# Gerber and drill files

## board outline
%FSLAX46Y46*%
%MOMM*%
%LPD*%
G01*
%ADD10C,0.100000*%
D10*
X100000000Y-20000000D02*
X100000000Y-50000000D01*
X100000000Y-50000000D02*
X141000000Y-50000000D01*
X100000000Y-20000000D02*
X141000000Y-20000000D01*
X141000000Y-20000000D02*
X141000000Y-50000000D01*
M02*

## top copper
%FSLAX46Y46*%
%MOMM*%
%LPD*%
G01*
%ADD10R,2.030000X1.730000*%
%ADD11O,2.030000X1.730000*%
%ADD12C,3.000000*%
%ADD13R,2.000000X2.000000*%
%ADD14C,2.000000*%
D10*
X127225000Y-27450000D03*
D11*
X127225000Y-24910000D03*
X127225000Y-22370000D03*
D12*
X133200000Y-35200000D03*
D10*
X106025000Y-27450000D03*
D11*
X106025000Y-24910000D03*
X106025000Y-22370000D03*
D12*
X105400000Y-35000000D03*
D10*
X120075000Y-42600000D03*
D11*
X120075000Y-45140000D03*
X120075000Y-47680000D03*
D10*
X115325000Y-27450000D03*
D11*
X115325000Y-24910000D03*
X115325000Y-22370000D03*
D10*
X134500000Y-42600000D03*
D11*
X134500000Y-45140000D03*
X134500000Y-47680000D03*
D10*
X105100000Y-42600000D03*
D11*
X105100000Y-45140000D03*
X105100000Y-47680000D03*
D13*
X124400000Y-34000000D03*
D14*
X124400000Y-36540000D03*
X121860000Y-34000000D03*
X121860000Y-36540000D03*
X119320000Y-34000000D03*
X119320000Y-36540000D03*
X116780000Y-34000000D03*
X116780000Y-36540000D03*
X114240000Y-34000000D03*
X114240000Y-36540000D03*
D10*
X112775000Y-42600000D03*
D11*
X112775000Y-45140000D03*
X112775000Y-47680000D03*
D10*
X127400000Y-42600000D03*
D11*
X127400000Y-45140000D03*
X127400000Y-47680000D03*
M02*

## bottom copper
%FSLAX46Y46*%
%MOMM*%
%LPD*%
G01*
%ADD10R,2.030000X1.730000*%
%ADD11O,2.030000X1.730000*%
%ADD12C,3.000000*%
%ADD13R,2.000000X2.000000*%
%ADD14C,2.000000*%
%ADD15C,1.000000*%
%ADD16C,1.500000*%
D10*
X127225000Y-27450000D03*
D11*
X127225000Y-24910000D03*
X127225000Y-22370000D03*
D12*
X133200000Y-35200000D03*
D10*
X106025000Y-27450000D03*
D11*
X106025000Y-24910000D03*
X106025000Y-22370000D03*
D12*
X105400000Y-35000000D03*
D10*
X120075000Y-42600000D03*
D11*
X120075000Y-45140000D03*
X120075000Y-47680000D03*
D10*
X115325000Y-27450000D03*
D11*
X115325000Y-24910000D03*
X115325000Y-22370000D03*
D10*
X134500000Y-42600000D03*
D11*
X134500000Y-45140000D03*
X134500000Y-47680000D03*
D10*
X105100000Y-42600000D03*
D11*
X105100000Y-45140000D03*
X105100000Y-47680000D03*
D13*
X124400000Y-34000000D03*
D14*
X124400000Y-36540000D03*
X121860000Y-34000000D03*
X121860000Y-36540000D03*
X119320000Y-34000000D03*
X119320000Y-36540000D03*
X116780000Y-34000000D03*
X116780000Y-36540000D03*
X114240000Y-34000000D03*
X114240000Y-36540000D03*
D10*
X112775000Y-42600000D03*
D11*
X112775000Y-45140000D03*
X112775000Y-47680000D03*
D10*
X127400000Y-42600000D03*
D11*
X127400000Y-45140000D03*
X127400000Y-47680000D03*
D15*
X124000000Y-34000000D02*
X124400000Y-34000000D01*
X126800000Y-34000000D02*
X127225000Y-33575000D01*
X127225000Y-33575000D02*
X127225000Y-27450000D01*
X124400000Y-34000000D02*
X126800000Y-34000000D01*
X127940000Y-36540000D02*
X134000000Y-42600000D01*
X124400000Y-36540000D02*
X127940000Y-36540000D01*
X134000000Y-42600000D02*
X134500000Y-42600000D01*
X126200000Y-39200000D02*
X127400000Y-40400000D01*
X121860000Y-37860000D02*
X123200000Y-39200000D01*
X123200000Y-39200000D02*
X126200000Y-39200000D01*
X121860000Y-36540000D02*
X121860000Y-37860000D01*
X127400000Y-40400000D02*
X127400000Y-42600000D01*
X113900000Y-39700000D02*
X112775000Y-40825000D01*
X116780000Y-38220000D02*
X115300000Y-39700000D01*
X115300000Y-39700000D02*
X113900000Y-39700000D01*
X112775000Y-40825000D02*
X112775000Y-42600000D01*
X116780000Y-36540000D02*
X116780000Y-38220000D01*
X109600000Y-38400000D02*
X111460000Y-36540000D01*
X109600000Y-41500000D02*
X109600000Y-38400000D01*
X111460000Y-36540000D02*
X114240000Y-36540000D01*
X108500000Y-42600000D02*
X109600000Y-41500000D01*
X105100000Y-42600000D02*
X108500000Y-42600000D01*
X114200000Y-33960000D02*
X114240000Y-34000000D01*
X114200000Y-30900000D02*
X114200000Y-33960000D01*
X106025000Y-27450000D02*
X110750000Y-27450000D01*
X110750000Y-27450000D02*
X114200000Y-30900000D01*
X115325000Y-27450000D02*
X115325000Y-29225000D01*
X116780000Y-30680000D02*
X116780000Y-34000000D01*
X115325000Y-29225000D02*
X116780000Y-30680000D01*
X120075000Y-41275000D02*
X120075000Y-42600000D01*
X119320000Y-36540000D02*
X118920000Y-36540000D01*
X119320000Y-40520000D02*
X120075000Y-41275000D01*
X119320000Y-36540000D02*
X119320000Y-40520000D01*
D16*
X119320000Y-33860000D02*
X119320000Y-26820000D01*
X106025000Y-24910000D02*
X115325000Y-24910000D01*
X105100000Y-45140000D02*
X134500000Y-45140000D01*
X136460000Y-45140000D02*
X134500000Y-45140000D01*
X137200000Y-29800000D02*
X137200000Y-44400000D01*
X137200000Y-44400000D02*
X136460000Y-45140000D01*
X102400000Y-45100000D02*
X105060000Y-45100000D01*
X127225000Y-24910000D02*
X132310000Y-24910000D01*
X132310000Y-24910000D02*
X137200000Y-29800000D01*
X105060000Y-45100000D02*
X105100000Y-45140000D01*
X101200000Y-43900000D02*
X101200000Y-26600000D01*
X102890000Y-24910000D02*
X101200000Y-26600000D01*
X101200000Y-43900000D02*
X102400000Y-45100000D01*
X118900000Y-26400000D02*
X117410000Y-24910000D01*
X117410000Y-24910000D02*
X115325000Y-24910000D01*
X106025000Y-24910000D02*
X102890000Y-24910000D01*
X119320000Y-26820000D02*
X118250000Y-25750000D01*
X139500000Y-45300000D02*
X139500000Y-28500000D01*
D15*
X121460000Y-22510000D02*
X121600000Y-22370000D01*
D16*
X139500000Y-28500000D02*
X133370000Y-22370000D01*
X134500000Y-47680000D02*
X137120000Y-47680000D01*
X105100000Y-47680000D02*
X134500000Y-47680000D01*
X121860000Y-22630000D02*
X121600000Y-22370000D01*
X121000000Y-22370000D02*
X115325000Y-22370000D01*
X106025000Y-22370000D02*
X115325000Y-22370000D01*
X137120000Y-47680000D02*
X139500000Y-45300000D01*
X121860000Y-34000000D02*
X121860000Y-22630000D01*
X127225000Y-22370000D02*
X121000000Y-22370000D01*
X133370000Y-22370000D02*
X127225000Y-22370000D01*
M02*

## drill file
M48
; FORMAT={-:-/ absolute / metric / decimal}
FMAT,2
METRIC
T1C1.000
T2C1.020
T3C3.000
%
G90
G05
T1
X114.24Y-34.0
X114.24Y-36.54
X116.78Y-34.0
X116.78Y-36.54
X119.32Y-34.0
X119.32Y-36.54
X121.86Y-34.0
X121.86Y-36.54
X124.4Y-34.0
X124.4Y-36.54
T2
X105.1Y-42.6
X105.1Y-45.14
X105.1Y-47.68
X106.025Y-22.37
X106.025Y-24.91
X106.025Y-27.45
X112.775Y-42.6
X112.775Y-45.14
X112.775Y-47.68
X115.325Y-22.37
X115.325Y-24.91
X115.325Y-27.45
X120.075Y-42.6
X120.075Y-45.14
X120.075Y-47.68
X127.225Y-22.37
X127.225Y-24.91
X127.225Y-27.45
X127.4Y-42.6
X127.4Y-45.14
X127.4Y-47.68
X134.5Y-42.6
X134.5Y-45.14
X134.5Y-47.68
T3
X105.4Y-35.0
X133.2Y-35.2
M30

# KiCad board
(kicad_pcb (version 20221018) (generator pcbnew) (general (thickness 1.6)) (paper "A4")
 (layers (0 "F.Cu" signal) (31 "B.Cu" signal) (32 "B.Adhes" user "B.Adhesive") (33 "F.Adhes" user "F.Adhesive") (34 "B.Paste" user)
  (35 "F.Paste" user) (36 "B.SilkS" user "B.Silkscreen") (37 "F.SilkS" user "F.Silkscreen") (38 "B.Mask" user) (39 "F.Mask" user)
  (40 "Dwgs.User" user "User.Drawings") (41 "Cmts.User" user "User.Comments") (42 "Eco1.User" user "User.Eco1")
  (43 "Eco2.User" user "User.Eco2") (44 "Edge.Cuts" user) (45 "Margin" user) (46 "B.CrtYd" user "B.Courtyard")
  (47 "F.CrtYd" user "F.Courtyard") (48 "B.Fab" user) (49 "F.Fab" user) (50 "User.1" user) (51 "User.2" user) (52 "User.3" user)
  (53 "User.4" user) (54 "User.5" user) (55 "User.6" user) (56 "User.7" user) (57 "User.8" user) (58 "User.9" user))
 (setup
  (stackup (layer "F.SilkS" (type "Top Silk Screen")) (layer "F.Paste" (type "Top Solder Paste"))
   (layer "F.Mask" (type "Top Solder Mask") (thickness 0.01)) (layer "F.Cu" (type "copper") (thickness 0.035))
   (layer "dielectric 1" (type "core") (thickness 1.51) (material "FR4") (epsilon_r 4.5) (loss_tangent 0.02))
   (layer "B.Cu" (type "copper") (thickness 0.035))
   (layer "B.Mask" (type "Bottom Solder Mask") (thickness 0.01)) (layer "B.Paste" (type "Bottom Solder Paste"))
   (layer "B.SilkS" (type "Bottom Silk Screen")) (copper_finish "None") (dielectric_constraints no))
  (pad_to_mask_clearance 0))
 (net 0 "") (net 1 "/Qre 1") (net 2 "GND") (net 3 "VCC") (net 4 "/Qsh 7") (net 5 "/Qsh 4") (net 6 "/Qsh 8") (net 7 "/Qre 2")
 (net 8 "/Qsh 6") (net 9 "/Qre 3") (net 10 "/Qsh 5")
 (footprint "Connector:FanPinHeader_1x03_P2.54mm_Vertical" (layer "F.Cu") (at 127.225 27.45 90)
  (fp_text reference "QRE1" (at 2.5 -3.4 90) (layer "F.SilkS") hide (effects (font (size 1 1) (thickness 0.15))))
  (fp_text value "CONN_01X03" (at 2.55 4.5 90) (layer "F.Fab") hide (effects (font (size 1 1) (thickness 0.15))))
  (pad "1" thru_hole rect (at 0 0 180) (size 2.03 1.73) (drill 1.02) (layers "*.Cu" "*.Mask") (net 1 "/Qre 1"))
  (pad "2" thru_hole oval (at 2.54 0 180) (size 2.03 1.73) (drill 1.02) (layers "*.Cu" "*.Mask") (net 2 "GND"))
  (pad "3" thru_hole oval (at 5.08 0 180) (size 2.03 1.73) (drill 1.02) (layers "*.Cu" "*.Mask") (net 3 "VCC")))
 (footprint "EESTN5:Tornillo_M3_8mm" (layer "F.Cu") (at 133.2 35.2)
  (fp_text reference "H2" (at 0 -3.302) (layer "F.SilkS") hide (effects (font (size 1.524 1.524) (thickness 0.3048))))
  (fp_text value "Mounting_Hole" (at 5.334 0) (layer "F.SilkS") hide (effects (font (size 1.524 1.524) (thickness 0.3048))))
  (pad "1" thru_hole circle (at 0 0) (size 3 3) (drill 3) (layers "*.Cu" "F.SilkS")))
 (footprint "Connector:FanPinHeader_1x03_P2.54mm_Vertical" (layer "F.Cu") (at 106.025 27.45 90)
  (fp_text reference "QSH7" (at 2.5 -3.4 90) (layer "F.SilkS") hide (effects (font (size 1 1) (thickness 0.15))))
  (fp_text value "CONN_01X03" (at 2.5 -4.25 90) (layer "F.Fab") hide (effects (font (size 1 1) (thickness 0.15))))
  (pad "1" thru_hole rect (at 0 0 180) (size 2.03 1.73) (drill 1.02) (layers "*.Cu" "*.Mask") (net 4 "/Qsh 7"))
  (pad "2" thru_hole oval (at 2.54 0 180) (size 2.03 1.73) (drill 1.02) (layers "*.Cu" "*.Mask") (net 2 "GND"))
  (pad "3" thru_hole oval (at 5.08 0 180) (size 2.03 1.73) (drill 1.02) (layers "*.Cu" "*.Mask") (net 3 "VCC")))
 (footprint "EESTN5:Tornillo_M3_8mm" (layer "F.Cu") (at 105.4 35)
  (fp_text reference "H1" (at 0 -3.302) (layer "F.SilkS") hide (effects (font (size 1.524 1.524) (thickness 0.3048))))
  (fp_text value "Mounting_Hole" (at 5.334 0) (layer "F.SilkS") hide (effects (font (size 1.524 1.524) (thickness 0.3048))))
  (pad "1" thru_hole circle (at 0 0) (size 3 3) (drill 3) (layers "*.Cu" "F.SilkS")))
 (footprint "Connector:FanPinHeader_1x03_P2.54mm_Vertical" (layer "F.Cu") (at 120.075 42.6 -90)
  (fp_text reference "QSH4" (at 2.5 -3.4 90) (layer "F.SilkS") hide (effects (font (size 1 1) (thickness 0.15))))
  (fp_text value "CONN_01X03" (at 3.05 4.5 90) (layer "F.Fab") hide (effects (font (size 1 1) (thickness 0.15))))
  (pad "1" thru_hole rect (at 0 0) (size 2.03 1.73) (drill 1.02) (layers "*.Cu" "*.Mask") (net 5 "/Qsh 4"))
  (pad "2" thru_hole oval (at 2.54 0) (size 2.03 1.73) (drill 1.02) (layers "*.Cu" "*.Mask") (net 2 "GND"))
  (pad "3" thru_hole oval (at 5.08 0) (size 2.03 1.73) (drill 1.02) (layers "*.Cu" "*.Mask") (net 3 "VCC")))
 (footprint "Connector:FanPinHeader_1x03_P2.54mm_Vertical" (layer "F.Cu") (at 115.325 27.45 90)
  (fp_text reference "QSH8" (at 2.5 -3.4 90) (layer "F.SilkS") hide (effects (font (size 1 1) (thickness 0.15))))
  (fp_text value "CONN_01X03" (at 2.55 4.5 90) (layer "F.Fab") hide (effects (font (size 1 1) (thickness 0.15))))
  (pad "1" thru_hole rect (at 0 0 180) (size 2.03 1.73) (drill 1.02) (layers "*.Cu" "*.Mask") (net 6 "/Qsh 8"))
  (pad "2" thru_hole oval (at 2.54 0 180) (size 2.03 1.73) (drill 1.02) (layers "*.Cu" "*.Mask") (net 2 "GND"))
  (pad "3" thru_hole oval (at 5.08 0 180) (size 2.03 1.73) (drill 1.02) (layers "*.Cu" "*.Mask") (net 3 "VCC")))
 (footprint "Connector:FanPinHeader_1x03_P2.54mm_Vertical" (layer "F.Cu") (at 134.5 42.6 -90)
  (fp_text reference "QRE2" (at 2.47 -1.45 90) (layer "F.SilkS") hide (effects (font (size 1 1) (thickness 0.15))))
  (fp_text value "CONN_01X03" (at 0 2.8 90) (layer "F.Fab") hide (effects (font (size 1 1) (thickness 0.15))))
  (pad "1" thru_hole rect (at 0 0) (size 2.03 1.73) (drill 1.02) (layers "*.Cu" "*.Mask") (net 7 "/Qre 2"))
  (pad "2" thru_hole oval (at 2.54 0) (size 2.03 1.73) (drill 1.02) (layers "*.Cu" "*.Mask") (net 2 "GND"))
  (pad "3" thru_hole oval (at 5.08 0) (size 2.03 1.73) (drill 1.02) (layers "*.Cu" "*.Mask") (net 3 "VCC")))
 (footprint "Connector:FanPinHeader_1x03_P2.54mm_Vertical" (layer "F.Cu") (at 105.1 42.6 -90)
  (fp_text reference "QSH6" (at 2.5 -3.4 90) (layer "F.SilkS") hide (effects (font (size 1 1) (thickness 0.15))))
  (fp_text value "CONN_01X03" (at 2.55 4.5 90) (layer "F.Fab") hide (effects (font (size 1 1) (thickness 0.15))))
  (pad "1" thru_hole rect (at 0 0) (size 2.03 1.73) (drill 1.02) (layers "*.Cu" "*.Mask") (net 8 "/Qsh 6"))
  (pad "2" thru_hole oval (at 2.54 0) (size 2.03 1.73) (drill 1.02) (layers "*.Cu" "*.Mask") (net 2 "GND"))
  (pad "3" thru_hole oval (at 5.08 0) (size 2.03 1.73) (drill 1.02) (layers "*.Cu" "*.Mask") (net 3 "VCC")))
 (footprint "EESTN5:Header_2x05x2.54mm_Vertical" (layer "F.Cu") (at 119.32 35.27 180)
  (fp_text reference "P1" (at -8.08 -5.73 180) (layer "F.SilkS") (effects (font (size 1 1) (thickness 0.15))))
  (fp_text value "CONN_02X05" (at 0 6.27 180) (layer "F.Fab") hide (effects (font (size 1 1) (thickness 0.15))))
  (pad "1" thru_hole rect (at -5.08 1.27 180) (size 2 2) (drill 1) (layers "*.Cu" "*.Mask") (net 1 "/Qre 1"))
  (pad "2" thru_hole circle (at -5.08 -1.27 180) (size 2 2) (drill 1) (layers "*.Cu" "*.Mask") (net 7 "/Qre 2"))
  (pad "3" thru_hole circle (at -2.54 1.27 180) (size 2 2) (drill 1) (layers "*.Cu" "*.Mask") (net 3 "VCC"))
  (pad "4" thru_hole circle (at -2.54 -1.27 180) (size 2 2) (drill 1) (layers "*.Cu" "*.Mask") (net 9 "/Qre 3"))
  (pad "5" thru_hole circle (at 0 1.27 180) (size 2 2) (drill 1) (layers "*.Cu" "*.Mask") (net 2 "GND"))
  (pad "6" thru_hole circle (at 0 -1.27 180) (size 2 2) (drill 1) (layers "*.Cu" "*.Mask") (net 5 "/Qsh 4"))
  (pad "7" thru_hole circle (at 2.54 1.27 180) (size 2 2) (drill 1) (layers "*.Cu" "*.Mask") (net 6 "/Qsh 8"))
  (pad "8" thru_hole circle (at 2.54 -1.27 180) (size 2 2) (drill 1) (layers "*.Cu" "*.Mask") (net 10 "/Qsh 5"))
  (pad "9" thru_hole circle (at 5.08 1.27 180) (size 2 2) (drill 1) (layers "*.Cu" "*.Mask") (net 4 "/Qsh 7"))
  (pad "10" thru_hole circle (at 5.08 -1.27 180) (size 2 2) (drill 1) (layers "*.Cu" "*.Mask") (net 8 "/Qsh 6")))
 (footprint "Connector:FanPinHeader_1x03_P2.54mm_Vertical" (layer "F.Cu") (at 112.775 42.6 -90)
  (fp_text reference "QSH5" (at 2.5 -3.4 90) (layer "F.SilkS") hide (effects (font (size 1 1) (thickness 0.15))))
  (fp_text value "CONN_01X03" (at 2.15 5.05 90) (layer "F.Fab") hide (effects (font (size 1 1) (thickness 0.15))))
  (pad "1" thru_hole rect (at 0 0) (size 2.03 1.73) (drill 1.02) (layers "*.Cu" "*.Mask") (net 10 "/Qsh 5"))
  (pad "2" thru_hole oval (at 2.54 0) (size 2.03 1.73) (drill 1.02) (layers "*.Cu" "*.Mask") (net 2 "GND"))
  (pad "3" thru_hole oval (at 5.08 0) (size 2.03 1.73) (drill 1.02) (layers "*.Cu" "*.Mask") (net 3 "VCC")))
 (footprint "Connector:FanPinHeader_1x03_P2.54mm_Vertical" (layer "F.Cu") (at 127.4 42.6 -90)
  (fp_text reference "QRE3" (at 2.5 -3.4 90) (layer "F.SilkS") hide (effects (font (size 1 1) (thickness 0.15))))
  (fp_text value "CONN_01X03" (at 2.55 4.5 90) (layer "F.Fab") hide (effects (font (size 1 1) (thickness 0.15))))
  (pad "1" thru_hole rect (at 0 0) (size 2.03 1.73) (drill 1.02) (layers "*.Cu" "*.Mask") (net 9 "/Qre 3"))
  (pad "2" thru_hole oval (at 2.54 0) (size 2.03 1.73) (drill 1.02) (layers "*.Cu" "*.Mask") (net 2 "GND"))
  (pad "3" thru_hole oval (at 5.08 0) (size 2.03 1.73) (drill 1.02) (layers "*.Cu" "*.Mask") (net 3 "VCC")))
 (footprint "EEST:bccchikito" (layer "B.Cu") (at 138.6 22.6 180)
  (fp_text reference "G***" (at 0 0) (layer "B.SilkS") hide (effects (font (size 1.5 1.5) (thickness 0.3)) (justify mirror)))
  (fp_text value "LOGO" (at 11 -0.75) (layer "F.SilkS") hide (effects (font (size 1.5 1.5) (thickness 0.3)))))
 (gr_line (start 100 20) (end 100 50) (stroke (width 0.1) (type default)) (layer "Edge.Cuts"))
 (gr_line (start 100 50) (end 141 50) (stroke (width 0.1) (type default)) (layer "Edge.Cuts"))
 (gr_line (start 100 20) (end 141 20) (stroke (width 0.1) (type default)) (layer "Edge.Cuts"))
 (gr_line (start 141 20) (end 141 50) (stroke (width 0.1) (type default)) (layer "Edge.Cuts"))
 (segment (start 124 34) (end 124.4 34) (width 1) (layer "B.Cu") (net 1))
 (segment (start 126.8 34) (end 127.225 33.575) (width 1) (layer "B.Cu") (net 1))
 (segment (start 127.225 33.575) (end 127.225 27.45) (width 1) (layer "B.Cu") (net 1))
 (segment (start 124.4 34) (end 126.8 34) (width 1) (layer "B.Cu") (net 1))
 (segment (start 127.94 36.54) (end 134 42.6) (width 1) (layer "B.Cu") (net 7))
 (segment (start 124.4 36.54) (end 127.94 36.54) (width 1) (layer "B.Cu") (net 7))
 (segment (start 134 42.6) (end 134.5 42.6) (width 1) (layer "B.Cu") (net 7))
 (segment (start 126.2 39.2) (end 127.4 40.4) (width 1) (layer "B.Cu") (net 9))
 (segment (start 121.86 37.86) (end 123.2 39.2) (width 1) (layer "B.Cu") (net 9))
 (segment (start 123.2 39.2) (end 126.2 39.2) (width 1) (layer "B.Cu") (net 9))
 (segment (start 121.86 36.54) (end 121.86 37.86) (width 1) (layer "B.Cu") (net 9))
 (segment (start 127.4 40.4) (end 127.4 42.6) (width 1) (layer "B.Cu") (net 9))
 (segment (start 113.9 39.7) (end 112.775 40.825) (width 1) (layer "B.Cu") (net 10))
 (segment (start 116.78 38.22) (end 115.3 39.7) (width 1) (layer "B.Cu") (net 10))
 (segment (start 115.3 39.7) (end 113.9 39.7) (width 1) (layer "B.Cu") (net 10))
 (segment (start 112.775 40.825) (end 112.775 42.6) (width 1) (layer "B.Cu") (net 10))
 (segment (start 116.78 36.54) (end 116.78 38.22) (width 1) (layer "B.Cu") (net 10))
 (segment (start 109.6 38.4) (end 111.46 36.54) (width 1) (layer "B.Cu") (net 8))
 (segment (start 109.6 41.5) (end 109.6 38.4) (width 1) (layer "B.Cu") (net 8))
 (segment (start 111.46 36.54) (end 114.24 36.54) (width 1) (layer "B.Cu") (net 8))
 (segment (start 108.5 42.6) (end 109.6 41.5) (width 1) (layer "B.Cu") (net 8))
 (segment (start 105.1 42.6) (end 108.5 42.6) (width 1) (layer "B.Cu") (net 8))
 (segment (start 114.2 33.96) (end 114.24 34) (width 1) (layer "B.Cu") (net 4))
 (segment (start 114.2 30.9) (end 114.2 33.96) (width 1) (layer "B.Cu") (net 4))
 (segment (start 106.025 27.45) (end 110.75 27.45) (width 1) (layer "B.Cu") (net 4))
 (segment (start 110.75 27.45) (end 114.2 30.9) (width 1) (layer "B.Cu") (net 4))
 (segment (start 115.325 27.45) (end 115.325 29.225) (width 1) (layer "B.Cu") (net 6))
 (segment (start 116.78 30.68) (end 116.78 34) (width 1) (layer "B.Cu") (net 6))
 (segment (start 115.325 29.225) (end 116.78 30.68) (width 1) (layer "B.Cu") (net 6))
 (segment (start 120.075 41.275) (end 120.075 42.6) (width 1) (layer "B.Cu") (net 5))
 (segment (start 119.32 36.54) (end 118.92 36.54) (width 1) (layer "B.Cu") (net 5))
 (segment (start 119.32 40.52) (end 120.075 41.275) (width 1) (layer "B.Cu") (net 5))
 (segment (start 119.32 36.54) (end 119.32 40.52) (width 1) (layer "B.Cu") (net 5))
 (segment (start 119.32 33.86) (end 119.32 26.82) (width 1.5) (layer "B.Cu") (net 2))
 (segment (start 106.025 24.91) (end 115.325 24.91) (width 1.5) (layer "B.Cu") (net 2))
 (segment (start 105.1 45.14) (end 134.5 45.14) (width 1.5) (layer "B.Cu") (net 2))
 (segment (start 136.46 45.14) (end 134.5 45.14) (width 1.5) (layer "B.Cu") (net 2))
 (segment (start 137.2 29.8) (end 137.2 44.4) (width 1.5) (layer "B.Cu") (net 2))
 (segment (start 137.2 44.4) (end 136.46 45.14) (width 1.5) (layer "B.Cu") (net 2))
 (segment (start 102.4 45.1) (end 105.06 45.1) (width 1.5) (layer "B.Cu") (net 2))
 (segment (start 127.225 24.91) (end 132.31 24.91) (width 1.5) (layer "B.Cu") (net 2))
 (segment (start 132.31 24.91) (end 137.2 29.8) (width 1.5) (layer "B.Cu") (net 2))
 (segment (start 105.06 45.1) (end 105.1 45.14) (width 1.5) (layer "B.Cu") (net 2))
 (segment (start 101.2 43.9) (end 101.2 26.6) (width 1.5) (layer "B.Cu") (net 2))
 (segment (start 102.89 24.91) (end 101.2 26.6) (width 1.5) (layer "B.Cu") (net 2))
 (segment (start 101.2 43.9) (end 102.4 45.1) (width 1.5) (layer "B.Cu") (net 2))
 (segment (start 118.9 26.4) (end 117.41 24.91) (width 1.5) (layer "B.Cu") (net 2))
 (segment (start 117.41 24.91) (end 115.325 24.91) (width 1.5) (layer "B.Cu") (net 2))
 (segment (start 106.025 24.91) (end 102.89 24.91) (width 1.5) (layer "B.Cu") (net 2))
 (segment (start 119.32 26.82) (end 118.25 25.75) (width 1.5) (layer "B.Cu") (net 2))
 (segment (start 139.5 45.3) (end 139.5 28.5) (width 1.5) (layer "B.Cu") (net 3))
 (segment (start 121.46 22.51) (end 121.6 22.37) (width 1) (layer "B.Cu") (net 3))
 (segment (start 139.5 28.5) (end 133.37 22.37) (width 1.5) (layer "B.Cu") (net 3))
 (segment (start 134.5 47.68) (end 137.12 47.68) (width 1.5) (layer "B.Cu") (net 3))
 (segment (start 105.1 47.68) (end 134.5 47.68) (width 1.5) (layer "B.Cu") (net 3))
 (segment (start 121.86 22.63) (end 121.6 22.37) (width 1.5) (layer "B.Cu") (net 3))
 (segment (start 121 22.37) (end 115.325 22.37) (width 1.5) (layer "B.Cu") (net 3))
 (segment (start 106.025 22.37) (end 115.325 22.37) (width 1.5) (layer "B.Cu") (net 3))
 (segment (start 137.12 47.68) (end 139.5 45.3) (width 1.5) (layer "B.Cu") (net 3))
 (segment (start 121.86 34) (end 121.86 22.63) (width 1.5) (layer "B.Cu") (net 3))
 (segment (start 127.225 22.37) (end 121 22.37) (width 1.5) (layer "B.Cu") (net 3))
 (segment (start 133.37 22.37) (end 127.225 22.37) (width 1.5) (layer "B.Cu") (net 3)))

